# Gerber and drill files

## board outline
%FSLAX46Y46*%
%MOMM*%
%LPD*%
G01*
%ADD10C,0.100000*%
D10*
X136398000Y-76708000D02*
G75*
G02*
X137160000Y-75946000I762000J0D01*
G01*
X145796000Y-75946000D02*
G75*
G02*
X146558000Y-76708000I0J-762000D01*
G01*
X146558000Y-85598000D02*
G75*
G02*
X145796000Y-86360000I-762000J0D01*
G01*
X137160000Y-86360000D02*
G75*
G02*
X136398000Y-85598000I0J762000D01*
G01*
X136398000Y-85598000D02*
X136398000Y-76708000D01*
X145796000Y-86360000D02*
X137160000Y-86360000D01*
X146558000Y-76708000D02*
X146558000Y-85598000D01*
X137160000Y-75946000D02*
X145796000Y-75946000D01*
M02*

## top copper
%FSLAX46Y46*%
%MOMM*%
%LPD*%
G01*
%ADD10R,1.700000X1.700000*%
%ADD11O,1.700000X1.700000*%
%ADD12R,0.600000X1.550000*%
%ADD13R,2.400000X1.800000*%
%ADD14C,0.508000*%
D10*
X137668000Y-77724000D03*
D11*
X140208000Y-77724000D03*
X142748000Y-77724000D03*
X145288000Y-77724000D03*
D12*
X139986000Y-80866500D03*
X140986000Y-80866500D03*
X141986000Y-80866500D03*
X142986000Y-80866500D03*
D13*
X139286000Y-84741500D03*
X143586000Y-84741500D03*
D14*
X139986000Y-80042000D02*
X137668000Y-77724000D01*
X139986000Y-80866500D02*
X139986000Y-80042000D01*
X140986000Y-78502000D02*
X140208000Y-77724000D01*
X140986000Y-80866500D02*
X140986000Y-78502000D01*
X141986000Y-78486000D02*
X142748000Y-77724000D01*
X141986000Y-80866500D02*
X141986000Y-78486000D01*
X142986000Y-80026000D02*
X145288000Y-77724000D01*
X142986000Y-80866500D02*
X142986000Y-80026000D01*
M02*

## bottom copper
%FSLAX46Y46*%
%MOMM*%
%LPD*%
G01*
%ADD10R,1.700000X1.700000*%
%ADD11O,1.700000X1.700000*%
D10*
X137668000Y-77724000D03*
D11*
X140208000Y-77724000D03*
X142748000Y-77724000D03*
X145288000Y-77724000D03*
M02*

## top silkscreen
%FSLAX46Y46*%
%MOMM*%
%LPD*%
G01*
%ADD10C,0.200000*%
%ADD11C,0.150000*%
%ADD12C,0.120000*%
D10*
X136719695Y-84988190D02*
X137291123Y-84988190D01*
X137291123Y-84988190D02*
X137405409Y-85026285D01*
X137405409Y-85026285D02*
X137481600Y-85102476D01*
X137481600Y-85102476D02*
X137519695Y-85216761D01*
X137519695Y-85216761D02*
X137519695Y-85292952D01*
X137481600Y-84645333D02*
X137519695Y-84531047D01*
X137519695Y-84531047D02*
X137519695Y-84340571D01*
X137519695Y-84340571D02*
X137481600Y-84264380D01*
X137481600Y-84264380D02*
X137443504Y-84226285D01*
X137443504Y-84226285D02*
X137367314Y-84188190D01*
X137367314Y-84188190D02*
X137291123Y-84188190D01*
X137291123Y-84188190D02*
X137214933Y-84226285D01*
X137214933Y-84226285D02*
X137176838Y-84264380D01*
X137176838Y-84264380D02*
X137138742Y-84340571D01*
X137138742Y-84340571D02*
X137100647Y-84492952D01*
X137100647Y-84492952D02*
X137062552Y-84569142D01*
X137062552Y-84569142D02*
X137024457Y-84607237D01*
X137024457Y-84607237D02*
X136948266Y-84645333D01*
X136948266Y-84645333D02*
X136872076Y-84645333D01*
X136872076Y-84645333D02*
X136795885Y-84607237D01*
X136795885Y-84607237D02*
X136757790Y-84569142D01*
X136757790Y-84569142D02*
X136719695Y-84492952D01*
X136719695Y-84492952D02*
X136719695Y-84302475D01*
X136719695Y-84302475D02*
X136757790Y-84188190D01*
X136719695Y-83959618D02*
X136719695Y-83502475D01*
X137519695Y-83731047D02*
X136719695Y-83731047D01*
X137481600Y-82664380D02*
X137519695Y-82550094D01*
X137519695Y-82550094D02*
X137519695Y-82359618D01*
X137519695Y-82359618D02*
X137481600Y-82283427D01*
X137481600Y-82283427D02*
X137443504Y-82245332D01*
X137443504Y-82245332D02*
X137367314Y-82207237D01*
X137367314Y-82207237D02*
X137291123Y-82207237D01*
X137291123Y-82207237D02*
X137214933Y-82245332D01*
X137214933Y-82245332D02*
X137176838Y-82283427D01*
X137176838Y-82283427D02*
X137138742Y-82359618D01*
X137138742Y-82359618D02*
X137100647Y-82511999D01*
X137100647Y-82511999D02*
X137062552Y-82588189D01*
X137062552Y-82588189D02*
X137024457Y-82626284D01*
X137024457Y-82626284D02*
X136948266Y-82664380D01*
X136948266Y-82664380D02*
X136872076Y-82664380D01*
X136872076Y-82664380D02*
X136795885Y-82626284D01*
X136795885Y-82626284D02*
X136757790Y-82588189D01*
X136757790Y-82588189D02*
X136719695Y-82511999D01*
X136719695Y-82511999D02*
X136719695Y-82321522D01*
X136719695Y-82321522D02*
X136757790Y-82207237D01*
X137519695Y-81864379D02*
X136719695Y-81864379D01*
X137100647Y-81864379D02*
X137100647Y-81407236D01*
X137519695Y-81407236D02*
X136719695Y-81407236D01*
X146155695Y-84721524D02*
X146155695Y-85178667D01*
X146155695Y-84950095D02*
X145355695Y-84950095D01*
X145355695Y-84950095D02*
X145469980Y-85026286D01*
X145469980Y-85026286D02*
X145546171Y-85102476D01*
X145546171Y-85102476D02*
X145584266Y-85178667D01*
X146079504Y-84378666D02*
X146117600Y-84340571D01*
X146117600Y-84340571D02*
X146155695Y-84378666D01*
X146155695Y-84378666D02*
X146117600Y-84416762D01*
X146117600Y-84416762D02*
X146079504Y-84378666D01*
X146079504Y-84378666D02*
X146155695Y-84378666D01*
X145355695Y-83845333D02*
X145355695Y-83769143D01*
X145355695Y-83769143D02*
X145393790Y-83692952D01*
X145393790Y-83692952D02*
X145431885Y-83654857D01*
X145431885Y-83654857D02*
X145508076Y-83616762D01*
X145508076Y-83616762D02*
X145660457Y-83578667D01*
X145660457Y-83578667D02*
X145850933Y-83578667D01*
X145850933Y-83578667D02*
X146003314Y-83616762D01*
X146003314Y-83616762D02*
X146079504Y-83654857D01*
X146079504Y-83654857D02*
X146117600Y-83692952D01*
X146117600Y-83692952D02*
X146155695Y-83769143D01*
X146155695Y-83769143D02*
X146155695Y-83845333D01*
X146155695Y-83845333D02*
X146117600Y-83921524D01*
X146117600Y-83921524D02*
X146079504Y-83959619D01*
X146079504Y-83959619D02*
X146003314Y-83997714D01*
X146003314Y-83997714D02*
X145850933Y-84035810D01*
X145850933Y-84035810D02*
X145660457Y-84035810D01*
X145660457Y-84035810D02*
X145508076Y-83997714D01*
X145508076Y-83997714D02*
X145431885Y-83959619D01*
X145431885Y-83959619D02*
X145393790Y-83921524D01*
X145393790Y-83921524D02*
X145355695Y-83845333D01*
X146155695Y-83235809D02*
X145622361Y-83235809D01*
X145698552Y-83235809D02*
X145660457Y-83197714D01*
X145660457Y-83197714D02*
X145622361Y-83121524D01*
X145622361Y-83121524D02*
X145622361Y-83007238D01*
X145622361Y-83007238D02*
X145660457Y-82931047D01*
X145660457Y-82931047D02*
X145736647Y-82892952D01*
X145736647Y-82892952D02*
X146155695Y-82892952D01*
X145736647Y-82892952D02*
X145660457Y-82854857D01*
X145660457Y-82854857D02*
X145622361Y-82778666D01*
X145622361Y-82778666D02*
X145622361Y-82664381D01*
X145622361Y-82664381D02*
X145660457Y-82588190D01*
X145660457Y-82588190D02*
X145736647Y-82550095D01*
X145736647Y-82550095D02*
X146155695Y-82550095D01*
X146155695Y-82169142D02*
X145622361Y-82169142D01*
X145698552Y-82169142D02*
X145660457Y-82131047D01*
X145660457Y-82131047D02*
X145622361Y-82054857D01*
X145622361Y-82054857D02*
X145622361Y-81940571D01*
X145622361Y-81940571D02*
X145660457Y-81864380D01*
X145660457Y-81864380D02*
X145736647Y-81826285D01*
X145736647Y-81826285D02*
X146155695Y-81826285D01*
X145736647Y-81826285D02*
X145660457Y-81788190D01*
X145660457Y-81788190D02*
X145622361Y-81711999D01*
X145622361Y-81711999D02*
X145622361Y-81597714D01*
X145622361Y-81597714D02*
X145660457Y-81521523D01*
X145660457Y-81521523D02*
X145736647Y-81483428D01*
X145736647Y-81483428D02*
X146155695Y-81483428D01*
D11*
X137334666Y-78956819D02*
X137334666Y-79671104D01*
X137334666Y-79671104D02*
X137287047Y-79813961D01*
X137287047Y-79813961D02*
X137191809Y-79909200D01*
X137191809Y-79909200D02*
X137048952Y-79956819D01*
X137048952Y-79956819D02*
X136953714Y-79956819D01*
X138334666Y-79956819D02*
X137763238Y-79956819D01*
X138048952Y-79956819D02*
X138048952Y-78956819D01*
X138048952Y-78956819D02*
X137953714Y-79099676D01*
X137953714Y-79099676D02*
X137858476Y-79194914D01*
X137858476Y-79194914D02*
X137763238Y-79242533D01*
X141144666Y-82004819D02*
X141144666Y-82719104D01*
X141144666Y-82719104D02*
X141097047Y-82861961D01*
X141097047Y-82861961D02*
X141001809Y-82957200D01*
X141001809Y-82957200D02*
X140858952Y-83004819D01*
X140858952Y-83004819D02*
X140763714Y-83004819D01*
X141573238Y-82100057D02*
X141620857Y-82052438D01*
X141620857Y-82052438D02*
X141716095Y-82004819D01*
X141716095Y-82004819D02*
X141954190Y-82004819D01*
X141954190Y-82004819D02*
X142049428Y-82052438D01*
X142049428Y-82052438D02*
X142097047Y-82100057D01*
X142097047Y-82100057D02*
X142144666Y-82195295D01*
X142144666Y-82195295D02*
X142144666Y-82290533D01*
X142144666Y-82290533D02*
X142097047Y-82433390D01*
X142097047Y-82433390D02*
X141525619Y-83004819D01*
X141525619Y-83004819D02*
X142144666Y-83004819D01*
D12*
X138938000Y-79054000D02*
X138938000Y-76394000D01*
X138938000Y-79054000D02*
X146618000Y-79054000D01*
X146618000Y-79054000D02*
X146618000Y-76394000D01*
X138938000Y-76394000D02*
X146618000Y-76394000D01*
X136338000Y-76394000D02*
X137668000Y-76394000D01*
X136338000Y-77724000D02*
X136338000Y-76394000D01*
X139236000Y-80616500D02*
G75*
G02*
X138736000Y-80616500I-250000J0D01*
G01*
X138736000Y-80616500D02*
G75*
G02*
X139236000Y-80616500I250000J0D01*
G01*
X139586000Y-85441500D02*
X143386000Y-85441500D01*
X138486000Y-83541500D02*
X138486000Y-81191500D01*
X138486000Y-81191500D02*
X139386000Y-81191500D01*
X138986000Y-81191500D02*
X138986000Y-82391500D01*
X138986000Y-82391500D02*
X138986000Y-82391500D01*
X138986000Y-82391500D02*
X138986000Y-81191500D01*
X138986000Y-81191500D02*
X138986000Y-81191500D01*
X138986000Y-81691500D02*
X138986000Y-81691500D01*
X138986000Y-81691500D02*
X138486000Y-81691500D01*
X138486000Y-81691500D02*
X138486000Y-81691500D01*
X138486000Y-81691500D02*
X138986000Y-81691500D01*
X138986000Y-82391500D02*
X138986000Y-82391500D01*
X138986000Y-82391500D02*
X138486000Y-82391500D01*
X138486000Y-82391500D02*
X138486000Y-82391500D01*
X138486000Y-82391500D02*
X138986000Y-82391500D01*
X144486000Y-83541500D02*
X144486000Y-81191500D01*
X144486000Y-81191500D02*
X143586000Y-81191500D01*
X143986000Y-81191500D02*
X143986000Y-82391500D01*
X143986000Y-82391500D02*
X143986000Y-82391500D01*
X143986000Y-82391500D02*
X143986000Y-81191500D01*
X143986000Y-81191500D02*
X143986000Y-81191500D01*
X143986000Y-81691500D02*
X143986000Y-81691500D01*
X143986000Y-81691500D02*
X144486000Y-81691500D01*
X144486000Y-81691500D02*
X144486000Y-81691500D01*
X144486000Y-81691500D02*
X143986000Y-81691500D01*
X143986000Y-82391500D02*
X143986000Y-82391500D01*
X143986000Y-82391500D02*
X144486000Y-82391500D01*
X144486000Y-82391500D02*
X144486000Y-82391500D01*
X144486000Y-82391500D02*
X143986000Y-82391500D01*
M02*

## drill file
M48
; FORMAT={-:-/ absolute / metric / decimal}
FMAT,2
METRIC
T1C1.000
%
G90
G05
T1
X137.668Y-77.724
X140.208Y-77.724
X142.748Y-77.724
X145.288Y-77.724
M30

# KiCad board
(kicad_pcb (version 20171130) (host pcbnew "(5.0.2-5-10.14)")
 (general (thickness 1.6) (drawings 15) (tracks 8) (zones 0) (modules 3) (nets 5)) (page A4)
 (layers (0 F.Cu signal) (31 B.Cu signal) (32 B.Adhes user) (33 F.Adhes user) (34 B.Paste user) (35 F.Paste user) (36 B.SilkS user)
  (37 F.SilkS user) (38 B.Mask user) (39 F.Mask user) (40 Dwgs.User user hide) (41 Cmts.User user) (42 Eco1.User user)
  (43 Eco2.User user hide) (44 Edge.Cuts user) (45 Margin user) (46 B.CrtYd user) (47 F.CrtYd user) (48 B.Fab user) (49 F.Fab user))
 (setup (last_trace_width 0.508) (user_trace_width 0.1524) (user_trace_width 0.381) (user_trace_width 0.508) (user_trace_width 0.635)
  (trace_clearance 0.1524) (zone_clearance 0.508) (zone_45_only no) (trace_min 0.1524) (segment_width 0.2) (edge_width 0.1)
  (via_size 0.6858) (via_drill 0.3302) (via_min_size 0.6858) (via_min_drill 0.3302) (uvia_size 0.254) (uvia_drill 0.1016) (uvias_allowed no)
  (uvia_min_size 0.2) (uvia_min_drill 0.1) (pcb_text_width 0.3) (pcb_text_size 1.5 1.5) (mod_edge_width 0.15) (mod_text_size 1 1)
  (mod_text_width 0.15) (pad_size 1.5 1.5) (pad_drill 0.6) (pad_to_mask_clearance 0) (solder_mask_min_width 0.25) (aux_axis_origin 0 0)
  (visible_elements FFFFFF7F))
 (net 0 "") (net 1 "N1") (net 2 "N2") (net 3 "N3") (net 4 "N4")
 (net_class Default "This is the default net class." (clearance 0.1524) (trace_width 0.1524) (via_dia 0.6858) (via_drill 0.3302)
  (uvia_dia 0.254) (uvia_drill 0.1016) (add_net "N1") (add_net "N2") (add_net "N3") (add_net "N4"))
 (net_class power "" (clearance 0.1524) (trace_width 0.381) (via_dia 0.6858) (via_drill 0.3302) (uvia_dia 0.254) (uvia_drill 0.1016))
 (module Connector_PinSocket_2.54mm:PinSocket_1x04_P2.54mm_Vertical (layer F.Cu) (at 137.668 77.724 90)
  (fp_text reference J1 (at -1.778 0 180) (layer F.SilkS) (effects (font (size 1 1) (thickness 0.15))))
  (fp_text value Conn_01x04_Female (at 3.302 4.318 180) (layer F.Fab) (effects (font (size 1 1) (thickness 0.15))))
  (fp_line (start -1.33 1.27) (end 1.33 1.27) (layer F.SilkS) (width 0.12))
  (fp_line (start -1.33 1.27) (end -1.33 8.95) (layer F.SilkS) (width 0.12))
  (fp_line (start -1.33 8.95) (end 1.33 8.95) (layer F.SilkS) (width 0.12))
  (fp_line (start 1.33 1.27) (end 1.33 8.95) (layer F.SilkS) (width 0.12))
  (fp_line (start 1.33 -1.33) (end 1.33 0) (layer F.SilkS) (width 0.12))
  (fp_line (start 0 -1.33) (end 1.33 -1.33) (layer F.SilkS) (width 0.12))
  (pad 1 thru_hole rect (at 0 0 90) (size 1.7 1.7) (drill 1) (layers *.Cu *.Mask) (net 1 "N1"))
  (pad 2 thru_hole oval (at 0 2.54 90) (size 1.7 1.7) (drill 1) (layers *.Cu *.Mask) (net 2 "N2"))
  (pad 3 thru_hole oval (at 0 5.08 90) (size 1.7 1.7) (drill 1) (layers *.Cu *.Mask) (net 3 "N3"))
  (pad 4 thru_hole oval (at 0 7.62 90) (size 1.7 1.7) (drill 1) (layers *.Cu *.Mask) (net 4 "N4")))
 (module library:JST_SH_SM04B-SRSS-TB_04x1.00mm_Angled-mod (layer F.Cu) (at 141.486 82.804)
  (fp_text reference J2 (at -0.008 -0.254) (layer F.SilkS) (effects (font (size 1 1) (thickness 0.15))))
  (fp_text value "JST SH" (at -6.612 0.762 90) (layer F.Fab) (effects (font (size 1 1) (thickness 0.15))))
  (fp_circle (center -2.5 -2.1875) (end -2.25 -2.1875) (layer F.SilkS) (width 0.12))
  (fp_line (start -1.9 2.6375) (end 1.9 2.6375) (layer F.SilkS) (width 0.12))
  (fp_line (start -3 0.7375) (end -3 -1.6125) (layer F.SilkS) (width 0.12))
  (fp_line (start -3 -1.6125) (end -2.1 -1.6125) (layer F.SilkS) (width 0.12))
  (fp_line (start -2.5 -1.6125) (end -2.5 -0.4125) (layer F.SilkS) (width 0.12))
  (fp_line (start -2.5 -0.4125) (end -2.5 -0.4125) (layer F.SilkS) (width 0.12))
  (fp_line (start -2.5 -0.4125) (end -2.5 -1.6125) (layer F.SilkS) (width 0.12))
  (fp_line (start -2.5 -1.6125) (end -2.5 -1.6125) (layer F.SilkS) (width 0.12))
  (fp_line (start -2.5 -1.1125) (end -2.5 -1.1125) (layer F.SilkS) (width 0.12))
  (fp_line (start -2.5 -1.1125) (end -3 -1.1125) (layer F.SilkS) (width 0.12))
  (fp_line (start -3 -1.1125) (end -3 -1.1125) (layer F.SilkS) (width 0.12))
  (fp_line (start -3 -1.1125) (end -2.5 -1.1125) (layer F.SilkS) (width 0.12))
  (fp_line (start -2.5 -0.4125) (end -2.5 -0.4125) (layer F.SilkS) (width 0.12))
  (fp_line (start -2.5 -0.4125) (end -3 -0.4125) (layer F.SilkS) (width 0.12))
  (fp_line (start -3 -0.4125) (end -3 -0.4125) (layer F.SilkS) (width 0.12))
  (fp_line (start -3 -0.4125) (end -2.5 -0.4125) (layer F.SilkS) (width 0.12))
  (fp_line (start 3 0.7375) (end 3 -1.6125) (layer F.SilkS) (width 0.12))
  (fp_line (start 3 -1.6125) (end 2.1 -1.6125) (layer F.SilkS) (width 0.12))
  (fp_line (start 2.5 -1.6125) (end 2.5 -0.4125) (layer F.SilkS) (width 0.12))
  (fp_line (start 2.5 -0.4125) (end 2.5 -0.4125) (layer F.SilkS) (width 0.12))
  (fp_line (start 2.5 -0.4125) (end 2.5 -1.6125) (layer F.SilkS) (width 0.12))
  (fp_line (start 2.5 -1.6125) (end 2.5 -1.6125) (layer F.SilkS) (width 0.12))
  (fp_line (start 2.5 -1.1125) (end 2.5 -1.1125) (layer F.SilkS) (width 0.12))
  (fp_line (start 2.5 -1.1125) (end 3 -1.1125) (layer F.SilkS) (width 0.12))
  (fp_line (start 3 -1.1125) (end 3 -1.1125) (layer F.SilkS) (width 0.12))
  (fp_line (start 3 -1.1125) (end 2.5 -1.1125) (layer F.SilkS) (width 0.12))
  (fp_line (start 2.5 -0.4125) (end 2.5 -0.4125) (layer F.SilkS) (width 0.12))
  (fp_line (start 2.5 -0.4125) (end 3 -0.4125) (layer F.SilkS) (width 0.12))
  (fp_line (start 3 -0.4125) (end 3 -0.4125) (layer F.SilkS) (width 0.12))
  (fp_line (start 3 -0.4125) (end 2.5 -0.4125) (layer F.SilkS) (width 0.12))
  (pad 1 smd rect (at -1.5 -1.9375) (size 0.6 1.55) (layers F.Cu F.Paste F.Mask) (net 1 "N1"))
  (pad 2 smd rect (at -0.5 -1.9375) (size 0.6 1.55) (layers F.Cu F.Paste F.Mask) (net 2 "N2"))
  (pad 3 smd rect (at 0.5 -1.9375) (size 0.6 1.55) (layers F.Cu F.Paste F.Mask) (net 3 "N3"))
  (pad 4 smd rect (at 1.5 -1.9375) (size 0.6 1.55) (layers F.Cu F.Paste F.Mask) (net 4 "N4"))
  (pad "" smd rect (at -2.2 1.9375) (size 2.4 1.8) (layers F.Cu F.Paste F.Mask))
  (pad "" smd rect (at 2.1 1.9375) (size 2.4 1.8) (layers F.Cu F.Paste F.Mask)))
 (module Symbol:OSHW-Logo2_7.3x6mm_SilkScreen (layer B.Cu) (at 140.208 81.534 180)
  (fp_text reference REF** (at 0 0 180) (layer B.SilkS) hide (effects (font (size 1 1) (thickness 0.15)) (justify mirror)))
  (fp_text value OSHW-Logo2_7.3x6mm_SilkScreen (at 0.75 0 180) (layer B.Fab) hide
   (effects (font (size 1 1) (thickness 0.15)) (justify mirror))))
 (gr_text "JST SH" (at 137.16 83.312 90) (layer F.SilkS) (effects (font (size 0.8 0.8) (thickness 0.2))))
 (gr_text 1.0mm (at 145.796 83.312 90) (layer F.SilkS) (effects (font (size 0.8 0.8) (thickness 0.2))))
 (gr_arc (start 137.16 76.708) (end 137.16 75.946) (angle -90) (layer Edge.Cuts) (width 0.1))
 (gr_arc (start 145.796 76.708) (end 146.558 76.708) (angle -90) (layer Edge.Cuts) (width 0.1))
 (gr_arc (start 145.796 85.598) (end 145.796 86.36) (angle -90) (layer Edge.Cuts) (width 0.1))
 (gr_arc (start 137.16 85.598) (end 136.398 85.598) (angle -90) (layer Edge.Cuts) (width 0.1))
 (gr_line (start 136.398 85.598) (end 136.398 76.708) (layer Edge.Cuts) (width 0.1))
 (gr_line (start 145.796 86.36) (end 137.16 86.36) (layer Edge.Cuts) (width 0.1))
 (gr_line (start 146.558 76.708) (end 146.558 85.598) (layer Edge.Cuts) (width 0.1))
 (gr_line (start 137.16 75.946) (end 145.796 75.946) (layer Edge.Cuts) (width 0.1))
 (segment (start 139.986 80.042) (end 137.668 77.724) (width 0.508) (layer F.Cu) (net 1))
 (segment (start 139.986 80.8665) (end 139.986 80.042) (width 0.508) (layer F.Cu) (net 1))
 (segment (start 140.986 78.502) (end 140.208 77.724) (width 0.508) (layer F.Cu) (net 2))
 (segment (start 140.986 80.8665) (end 140.986 78.502) (width 0.508) (layer F.Cu) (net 2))
 (segment (start 141.986 78.486) (end 142.748 77.724) (width 0.508) (layer F.Cu) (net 3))
 (segment (start 141.986 80.8665) (end 141.986 78.486) (width 0.508) (layer F.Cu) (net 3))
 (segment (start 142.986 80.026) (end 145.288 77.724) (width 0.508) (layer F.Cu) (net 4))
 (segment (start 142.986 80.8665) (end 142.986 80.026) (width 0.508) (layer F.Cu) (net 4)))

